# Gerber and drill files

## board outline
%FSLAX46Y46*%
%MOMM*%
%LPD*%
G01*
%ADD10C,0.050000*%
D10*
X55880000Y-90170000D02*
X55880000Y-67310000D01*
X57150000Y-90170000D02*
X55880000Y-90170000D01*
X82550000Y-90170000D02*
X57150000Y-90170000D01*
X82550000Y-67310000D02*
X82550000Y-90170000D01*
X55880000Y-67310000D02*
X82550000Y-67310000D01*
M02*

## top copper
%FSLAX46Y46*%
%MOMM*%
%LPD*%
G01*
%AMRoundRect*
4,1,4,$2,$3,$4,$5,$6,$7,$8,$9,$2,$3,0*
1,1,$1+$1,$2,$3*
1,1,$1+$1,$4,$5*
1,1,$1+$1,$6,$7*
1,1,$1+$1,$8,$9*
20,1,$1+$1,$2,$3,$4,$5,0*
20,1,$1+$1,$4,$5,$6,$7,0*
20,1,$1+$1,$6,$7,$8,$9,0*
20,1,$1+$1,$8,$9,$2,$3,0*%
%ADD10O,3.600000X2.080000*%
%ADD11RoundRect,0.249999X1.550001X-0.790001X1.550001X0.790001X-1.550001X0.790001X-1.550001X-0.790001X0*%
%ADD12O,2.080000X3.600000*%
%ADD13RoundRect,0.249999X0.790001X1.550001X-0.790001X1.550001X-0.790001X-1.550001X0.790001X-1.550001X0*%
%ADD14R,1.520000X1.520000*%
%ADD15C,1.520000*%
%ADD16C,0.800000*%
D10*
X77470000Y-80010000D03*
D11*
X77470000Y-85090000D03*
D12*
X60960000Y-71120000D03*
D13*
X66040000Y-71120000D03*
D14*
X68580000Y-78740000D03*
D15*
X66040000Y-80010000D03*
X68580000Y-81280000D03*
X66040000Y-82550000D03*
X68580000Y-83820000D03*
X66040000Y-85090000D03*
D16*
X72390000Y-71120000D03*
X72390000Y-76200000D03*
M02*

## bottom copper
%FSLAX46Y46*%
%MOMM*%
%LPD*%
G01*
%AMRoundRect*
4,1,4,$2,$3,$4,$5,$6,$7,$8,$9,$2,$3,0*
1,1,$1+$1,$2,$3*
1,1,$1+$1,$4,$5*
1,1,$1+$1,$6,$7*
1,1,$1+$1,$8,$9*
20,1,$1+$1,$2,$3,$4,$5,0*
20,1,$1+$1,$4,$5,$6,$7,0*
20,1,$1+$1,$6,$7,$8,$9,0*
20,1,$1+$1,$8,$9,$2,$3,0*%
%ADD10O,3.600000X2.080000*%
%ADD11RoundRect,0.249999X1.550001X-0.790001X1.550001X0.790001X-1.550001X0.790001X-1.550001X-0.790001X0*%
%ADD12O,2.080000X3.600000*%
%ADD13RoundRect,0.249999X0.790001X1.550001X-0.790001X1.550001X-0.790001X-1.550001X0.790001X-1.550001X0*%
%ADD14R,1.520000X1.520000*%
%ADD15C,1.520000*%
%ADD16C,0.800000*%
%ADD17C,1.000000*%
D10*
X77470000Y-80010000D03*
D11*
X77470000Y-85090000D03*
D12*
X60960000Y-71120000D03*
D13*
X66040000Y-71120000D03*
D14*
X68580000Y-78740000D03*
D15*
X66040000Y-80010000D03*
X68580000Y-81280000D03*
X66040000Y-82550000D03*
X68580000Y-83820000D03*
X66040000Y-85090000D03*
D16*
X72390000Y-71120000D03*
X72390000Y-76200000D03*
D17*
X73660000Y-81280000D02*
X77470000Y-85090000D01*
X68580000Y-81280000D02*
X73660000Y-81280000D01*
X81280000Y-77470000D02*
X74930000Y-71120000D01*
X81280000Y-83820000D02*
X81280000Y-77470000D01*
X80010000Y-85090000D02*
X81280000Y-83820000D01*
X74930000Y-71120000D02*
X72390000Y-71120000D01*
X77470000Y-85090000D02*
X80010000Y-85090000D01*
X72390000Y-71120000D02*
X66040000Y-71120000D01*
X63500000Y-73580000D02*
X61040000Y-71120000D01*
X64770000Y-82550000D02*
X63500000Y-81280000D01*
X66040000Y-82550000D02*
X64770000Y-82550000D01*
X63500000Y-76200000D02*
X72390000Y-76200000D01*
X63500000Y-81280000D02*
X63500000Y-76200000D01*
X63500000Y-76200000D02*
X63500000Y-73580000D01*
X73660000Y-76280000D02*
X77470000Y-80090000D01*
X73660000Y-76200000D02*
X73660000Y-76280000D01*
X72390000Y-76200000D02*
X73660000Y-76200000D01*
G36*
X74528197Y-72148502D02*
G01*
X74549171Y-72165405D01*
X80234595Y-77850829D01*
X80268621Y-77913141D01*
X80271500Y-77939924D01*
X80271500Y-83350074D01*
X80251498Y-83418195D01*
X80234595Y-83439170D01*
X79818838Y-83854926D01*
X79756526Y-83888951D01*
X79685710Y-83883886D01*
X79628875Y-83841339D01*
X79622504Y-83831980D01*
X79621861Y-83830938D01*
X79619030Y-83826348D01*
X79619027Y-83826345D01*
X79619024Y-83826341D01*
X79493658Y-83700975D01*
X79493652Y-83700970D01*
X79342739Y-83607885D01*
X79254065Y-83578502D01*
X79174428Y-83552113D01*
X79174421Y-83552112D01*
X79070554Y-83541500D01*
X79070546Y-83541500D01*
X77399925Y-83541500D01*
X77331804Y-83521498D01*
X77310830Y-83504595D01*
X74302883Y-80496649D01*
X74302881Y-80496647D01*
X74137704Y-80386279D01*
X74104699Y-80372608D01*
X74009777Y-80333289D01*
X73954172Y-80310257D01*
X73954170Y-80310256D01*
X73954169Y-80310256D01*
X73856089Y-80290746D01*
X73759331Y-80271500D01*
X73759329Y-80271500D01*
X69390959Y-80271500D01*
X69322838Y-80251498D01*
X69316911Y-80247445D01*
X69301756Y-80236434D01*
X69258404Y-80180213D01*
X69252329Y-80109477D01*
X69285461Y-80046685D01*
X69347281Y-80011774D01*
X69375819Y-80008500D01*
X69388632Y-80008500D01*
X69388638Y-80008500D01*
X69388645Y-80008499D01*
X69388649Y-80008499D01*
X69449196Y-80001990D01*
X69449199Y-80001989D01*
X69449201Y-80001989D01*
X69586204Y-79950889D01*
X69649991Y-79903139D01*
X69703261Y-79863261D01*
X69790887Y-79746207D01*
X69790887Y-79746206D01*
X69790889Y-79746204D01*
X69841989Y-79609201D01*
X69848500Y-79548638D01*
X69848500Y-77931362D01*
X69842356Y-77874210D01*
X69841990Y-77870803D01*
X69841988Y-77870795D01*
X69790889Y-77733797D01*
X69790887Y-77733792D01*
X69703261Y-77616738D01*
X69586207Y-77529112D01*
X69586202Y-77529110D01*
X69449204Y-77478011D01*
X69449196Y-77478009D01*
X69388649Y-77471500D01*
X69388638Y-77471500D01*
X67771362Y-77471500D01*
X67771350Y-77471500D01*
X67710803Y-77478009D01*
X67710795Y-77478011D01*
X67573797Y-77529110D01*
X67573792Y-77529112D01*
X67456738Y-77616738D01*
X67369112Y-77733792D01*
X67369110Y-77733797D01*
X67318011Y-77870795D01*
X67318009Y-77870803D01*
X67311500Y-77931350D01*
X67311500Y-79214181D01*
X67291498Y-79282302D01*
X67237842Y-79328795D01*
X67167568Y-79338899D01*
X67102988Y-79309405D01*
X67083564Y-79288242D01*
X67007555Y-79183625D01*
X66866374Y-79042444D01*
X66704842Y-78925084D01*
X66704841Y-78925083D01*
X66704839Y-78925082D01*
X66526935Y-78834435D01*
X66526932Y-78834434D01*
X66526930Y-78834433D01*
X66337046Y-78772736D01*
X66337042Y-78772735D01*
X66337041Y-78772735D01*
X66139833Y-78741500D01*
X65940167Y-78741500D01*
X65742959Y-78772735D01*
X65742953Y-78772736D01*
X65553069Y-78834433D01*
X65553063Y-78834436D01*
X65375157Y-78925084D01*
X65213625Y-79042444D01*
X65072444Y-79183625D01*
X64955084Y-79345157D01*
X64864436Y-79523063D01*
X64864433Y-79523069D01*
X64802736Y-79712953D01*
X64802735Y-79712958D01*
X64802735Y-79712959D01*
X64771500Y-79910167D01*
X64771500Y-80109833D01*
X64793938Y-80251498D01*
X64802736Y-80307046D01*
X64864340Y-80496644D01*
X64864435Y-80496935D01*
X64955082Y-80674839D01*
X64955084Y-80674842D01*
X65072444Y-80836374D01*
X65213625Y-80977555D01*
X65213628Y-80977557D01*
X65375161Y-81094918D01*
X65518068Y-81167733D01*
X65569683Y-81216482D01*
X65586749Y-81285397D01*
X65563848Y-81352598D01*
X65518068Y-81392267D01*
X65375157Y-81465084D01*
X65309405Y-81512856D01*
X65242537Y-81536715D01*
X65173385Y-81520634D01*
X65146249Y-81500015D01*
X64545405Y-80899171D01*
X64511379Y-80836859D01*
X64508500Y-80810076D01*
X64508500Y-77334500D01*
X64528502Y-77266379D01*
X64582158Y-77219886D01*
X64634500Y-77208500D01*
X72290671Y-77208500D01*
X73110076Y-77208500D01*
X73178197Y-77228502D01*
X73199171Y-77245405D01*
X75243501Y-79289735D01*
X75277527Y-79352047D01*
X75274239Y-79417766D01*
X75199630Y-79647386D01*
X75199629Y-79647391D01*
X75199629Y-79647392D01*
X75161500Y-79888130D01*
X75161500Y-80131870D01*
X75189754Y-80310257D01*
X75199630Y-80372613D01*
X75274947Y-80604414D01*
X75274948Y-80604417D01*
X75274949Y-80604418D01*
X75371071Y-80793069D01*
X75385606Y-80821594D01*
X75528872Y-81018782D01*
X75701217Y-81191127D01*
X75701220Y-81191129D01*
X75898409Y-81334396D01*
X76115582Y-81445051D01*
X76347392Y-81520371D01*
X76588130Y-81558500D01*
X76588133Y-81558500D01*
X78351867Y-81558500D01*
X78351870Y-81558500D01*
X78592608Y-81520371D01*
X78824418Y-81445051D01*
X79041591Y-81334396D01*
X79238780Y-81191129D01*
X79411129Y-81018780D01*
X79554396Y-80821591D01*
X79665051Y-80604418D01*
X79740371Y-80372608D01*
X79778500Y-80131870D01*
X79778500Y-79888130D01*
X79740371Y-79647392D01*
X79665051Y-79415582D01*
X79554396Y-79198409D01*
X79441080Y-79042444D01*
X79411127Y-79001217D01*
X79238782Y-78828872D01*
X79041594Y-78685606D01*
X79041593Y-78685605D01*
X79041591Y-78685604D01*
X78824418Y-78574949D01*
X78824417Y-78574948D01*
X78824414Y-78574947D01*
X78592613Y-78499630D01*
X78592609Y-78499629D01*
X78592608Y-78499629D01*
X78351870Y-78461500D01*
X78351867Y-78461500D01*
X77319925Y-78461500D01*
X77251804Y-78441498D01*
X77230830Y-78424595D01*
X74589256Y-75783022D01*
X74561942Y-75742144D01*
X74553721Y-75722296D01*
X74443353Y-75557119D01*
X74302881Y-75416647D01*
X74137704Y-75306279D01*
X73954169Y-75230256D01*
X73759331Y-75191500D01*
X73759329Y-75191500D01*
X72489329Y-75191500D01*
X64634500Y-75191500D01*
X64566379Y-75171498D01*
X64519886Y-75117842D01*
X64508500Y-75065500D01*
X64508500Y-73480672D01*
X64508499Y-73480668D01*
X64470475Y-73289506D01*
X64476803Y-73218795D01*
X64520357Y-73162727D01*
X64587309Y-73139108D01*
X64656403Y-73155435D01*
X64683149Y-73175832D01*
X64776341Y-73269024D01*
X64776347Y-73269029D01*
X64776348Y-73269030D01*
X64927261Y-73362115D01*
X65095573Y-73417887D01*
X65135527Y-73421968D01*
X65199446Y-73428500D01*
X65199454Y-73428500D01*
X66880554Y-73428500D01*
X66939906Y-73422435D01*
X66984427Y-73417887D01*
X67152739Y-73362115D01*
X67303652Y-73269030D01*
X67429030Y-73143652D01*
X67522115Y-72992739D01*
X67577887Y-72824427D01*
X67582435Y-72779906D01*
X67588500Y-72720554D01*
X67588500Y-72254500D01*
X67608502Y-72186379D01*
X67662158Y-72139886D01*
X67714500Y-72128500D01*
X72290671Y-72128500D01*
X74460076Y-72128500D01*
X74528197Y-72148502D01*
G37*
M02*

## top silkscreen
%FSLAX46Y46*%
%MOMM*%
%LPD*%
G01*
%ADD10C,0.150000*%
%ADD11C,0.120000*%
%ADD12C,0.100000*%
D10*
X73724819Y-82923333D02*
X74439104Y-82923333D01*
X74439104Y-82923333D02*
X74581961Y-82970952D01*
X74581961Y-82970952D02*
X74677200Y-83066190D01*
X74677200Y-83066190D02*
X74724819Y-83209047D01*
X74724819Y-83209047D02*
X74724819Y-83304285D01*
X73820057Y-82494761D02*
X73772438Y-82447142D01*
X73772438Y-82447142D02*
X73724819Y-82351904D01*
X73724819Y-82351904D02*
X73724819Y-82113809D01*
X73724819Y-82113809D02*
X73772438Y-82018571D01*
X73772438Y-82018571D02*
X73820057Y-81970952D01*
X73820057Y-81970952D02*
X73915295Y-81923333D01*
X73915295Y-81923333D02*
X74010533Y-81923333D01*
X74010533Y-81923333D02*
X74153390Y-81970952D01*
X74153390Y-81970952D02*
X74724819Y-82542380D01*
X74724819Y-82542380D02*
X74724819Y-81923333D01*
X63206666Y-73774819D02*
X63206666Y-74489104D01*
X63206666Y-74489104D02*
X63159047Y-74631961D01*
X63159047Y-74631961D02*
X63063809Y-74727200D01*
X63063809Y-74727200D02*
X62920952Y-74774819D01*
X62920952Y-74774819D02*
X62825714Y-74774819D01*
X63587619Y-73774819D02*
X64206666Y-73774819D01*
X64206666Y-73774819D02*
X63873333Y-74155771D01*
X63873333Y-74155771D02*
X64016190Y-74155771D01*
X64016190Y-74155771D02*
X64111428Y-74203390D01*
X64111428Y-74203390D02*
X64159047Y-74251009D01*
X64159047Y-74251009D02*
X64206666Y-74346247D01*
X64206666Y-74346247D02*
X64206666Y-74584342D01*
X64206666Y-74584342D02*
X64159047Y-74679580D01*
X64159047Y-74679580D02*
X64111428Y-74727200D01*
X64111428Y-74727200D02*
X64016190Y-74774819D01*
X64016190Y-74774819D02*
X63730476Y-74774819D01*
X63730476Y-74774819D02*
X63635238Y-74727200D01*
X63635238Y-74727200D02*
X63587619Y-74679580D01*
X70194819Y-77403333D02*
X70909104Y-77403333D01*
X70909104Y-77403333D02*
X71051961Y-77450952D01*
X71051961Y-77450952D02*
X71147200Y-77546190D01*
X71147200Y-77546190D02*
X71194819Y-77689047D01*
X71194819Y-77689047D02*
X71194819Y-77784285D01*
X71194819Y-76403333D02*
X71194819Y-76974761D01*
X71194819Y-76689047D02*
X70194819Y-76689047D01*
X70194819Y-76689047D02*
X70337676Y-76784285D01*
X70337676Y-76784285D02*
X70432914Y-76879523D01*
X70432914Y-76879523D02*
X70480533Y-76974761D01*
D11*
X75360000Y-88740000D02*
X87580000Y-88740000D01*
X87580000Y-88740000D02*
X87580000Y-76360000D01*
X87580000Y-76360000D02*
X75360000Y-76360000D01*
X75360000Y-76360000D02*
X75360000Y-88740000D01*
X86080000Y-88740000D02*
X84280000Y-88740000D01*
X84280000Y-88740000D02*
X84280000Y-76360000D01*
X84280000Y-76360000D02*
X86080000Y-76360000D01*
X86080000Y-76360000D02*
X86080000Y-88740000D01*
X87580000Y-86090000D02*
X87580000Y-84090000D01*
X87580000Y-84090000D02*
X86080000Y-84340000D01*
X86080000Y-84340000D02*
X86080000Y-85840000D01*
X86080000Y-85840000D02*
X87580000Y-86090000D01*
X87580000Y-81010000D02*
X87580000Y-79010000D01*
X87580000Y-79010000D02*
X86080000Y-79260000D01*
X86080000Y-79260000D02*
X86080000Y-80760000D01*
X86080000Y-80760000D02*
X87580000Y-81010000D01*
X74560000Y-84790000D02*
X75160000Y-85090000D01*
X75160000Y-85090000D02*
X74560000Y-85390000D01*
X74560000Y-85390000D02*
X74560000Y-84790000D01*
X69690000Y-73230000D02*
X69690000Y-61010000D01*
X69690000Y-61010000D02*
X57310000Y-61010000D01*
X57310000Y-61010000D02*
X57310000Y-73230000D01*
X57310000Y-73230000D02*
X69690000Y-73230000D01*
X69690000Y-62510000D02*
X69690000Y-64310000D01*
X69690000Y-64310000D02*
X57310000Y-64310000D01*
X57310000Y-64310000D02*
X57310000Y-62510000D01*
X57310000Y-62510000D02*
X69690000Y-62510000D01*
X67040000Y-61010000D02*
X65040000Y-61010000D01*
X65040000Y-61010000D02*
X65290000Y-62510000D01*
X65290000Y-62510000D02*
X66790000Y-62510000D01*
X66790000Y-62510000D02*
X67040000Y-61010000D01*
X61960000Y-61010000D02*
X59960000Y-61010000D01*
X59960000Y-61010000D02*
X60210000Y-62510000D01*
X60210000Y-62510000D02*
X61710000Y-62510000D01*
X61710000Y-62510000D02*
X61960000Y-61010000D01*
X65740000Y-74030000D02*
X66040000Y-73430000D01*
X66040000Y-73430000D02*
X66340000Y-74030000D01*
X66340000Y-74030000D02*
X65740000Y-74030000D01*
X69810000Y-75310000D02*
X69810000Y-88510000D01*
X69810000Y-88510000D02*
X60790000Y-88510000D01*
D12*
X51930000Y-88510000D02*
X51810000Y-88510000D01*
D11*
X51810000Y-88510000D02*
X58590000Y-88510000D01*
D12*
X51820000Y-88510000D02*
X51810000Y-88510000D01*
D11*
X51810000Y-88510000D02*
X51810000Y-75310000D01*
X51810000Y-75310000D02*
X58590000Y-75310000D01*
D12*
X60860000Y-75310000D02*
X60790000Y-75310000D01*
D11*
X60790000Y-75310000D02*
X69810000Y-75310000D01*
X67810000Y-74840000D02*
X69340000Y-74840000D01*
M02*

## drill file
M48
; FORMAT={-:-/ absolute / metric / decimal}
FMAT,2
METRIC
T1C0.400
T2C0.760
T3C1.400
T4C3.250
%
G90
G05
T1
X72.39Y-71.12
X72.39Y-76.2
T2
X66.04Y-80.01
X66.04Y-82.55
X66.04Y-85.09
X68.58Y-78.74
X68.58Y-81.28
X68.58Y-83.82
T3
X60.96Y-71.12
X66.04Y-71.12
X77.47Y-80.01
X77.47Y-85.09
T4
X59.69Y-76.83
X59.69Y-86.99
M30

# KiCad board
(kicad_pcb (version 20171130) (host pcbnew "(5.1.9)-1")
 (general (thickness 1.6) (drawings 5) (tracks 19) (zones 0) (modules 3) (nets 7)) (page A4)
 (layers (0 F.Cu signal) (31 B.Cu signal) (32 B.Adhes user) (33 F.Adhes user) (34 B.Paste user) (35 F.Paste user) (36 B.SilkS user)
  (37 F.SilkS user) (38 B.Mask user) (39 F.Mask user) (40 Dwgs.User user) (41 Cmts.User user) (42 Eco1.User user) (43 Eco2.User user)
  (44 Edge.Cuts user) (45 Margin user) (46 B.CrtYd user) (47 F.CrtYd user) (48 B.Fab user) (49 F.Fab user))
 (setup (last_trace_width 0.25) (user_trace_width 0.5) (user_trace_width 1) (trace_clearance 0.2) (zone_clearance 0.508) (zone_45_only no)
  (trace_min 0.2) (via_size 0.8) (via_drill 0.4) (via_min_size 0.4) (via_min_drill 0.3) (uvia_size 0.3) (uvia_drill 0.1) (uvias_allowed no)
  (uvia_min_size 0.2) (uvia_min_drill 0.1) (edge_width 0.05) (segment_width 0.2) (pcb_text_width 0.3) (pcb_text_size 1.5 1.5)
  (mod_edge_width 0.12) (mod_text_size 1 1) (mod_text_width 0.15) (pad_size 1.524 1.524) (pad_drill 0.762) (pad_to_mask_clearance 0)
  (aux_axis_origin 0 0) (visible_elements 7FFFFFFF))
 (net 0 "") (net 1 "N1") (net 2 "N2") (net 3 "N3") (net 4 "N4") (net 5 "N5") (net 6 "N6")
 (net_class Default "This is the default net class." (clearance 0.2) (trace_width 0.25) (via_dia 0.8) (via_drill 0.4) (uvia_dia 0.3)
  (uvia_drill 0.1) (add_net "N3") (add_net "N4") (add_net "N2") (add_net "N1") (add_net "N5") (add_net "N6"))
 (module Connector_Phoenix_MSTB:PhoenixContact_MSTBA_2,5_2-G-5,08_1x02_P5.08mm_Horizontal (layer F.Cu) (at 77.47 85.09 90)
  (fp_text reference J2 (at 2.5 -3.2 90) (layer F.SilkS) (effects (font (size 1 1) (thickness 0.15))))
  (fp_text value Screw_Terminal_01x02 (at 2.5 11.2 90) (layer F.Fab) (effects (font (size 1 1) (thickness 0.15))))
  (fp_line (start -3.65 -2.11) (end -3.65 10.11) (layer F.SilkS) (width 0.12))
  (fp_line (start -3.65 10.11) (end 8.73 10.11) (layer F.SilkS) (width 0.12))
  (fp_line (start 8.73 10.11) (end 8.73 -2.11) (layer F.SilkS) (width 0.12))
  (fp_line (start 8.73 -2.11) (end -3.65 -2.11) (layer F.SilkS) (width 0.12))
  (fp_line (start -3.65 8.61) (end -3.65 6.81) (layer F.SilkS) (width 0.12))
  (fp_line (start -3.65 6.81) (end 8.73 6.81) (layer F.SilkS) (width 0.12))
  (fp_line (start 8.73 6.81) (end 8.73 8.61) (layer F.SilkS) (width 0.12))
  (fp_line (start 8.73 8.61) (end -3.65 8.61) (layer F.SilkS) (width 0.12))
  (fp_line (start -1 10.11) (end 1 10.11) (layer F.SilkS) (width 0.12))
  (fp_line (start 1 10.11) (end 0.75 8.61) (layer F.SilkS) (width 0.12))
  (fp_line (start 0.75 8.61) (end -0.75 8.61) (layer F.SilkS) (width 0.12))
  (fp_line (start -0.75 8.61) (end -1 10.11) (layer F.SilkS) (width 0.12))
  (fp_line (start 4.08 10.11) (end 6.08 10.11) (layer F.SilkS) (width 0.12))
  (fp_line (start 6.08 10.11) (end 5.83 8.61) (layer F.SilkS) (width 0.12))
  (fp_line (start 5.83 8.61) (end 4.33 8.61) (layer F.SilkS) (width 0.12))
  (fp_line (start 4.33 8.61) (end 4.08 10.11) (layer F.SilkS) (width 0.12))
  (fp_line (start 0.3 -2.91) (end 0 -2.31) (layer F.SilkS) (width 0.12))
  (fp_line (start 0 -2.31) (end -0.3 -2.91) (layer F.SilkS) (width 0.12))
  (fp_line (start -0.3 -2.91) (end 0.3 -2.91) (layer F.SilkS) (width 0.12))
  (pad 2 thru_hole oval (at 5.08 0 90) (size 2.08 3.6) (drill 1.4) (layers *.Cu *.Mask) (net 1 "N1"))
  (pad 1 thru_hole roundrect (at 0 0 90) (size 2.08 3.6) (drill 1.4) (layers *.Cu *.Mask) (roundrect_rratio 0.120192) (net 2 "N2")))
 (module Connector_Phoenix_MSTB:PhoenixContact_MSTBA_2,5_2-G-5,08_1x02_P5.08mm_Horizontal (layer F.Cu) (at 66.04 71.12 180)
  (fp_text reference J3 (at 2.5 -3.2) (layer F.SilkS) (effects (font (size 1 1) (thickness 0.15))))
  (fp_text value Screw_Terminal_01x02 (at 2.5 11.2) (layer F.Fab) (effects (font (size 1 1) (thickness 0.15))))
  (fp_line (start -3.65 -2.11) (end -3.65 10.11) (layer F.SilkS) (width 0.12))
  (fp_line (start -3.65 10.11) (end 8.73 10.11) (layer F.SilkS) (width 0.12))
  (fp_line (start 8.73 10.11) (end 8.73 -2.11) (layer F.SilkS) (width 0.12))
  (fp_line (start 8.73 -2.11) (end -3.65 -2.11) (layer F.SilkS) (width 0.12))
  (fp_line (start -3.65 8.61) (end -3.65 6.81) (layer F.SilkS) (width 0.12))
  (fp_line (start -3.65 6.81) (end 8.73 6.81) (layer F.SilkS) (width 0.12))
  (fp_line (start 8.73 6.81) (end 8.73 8.61) (layer F.SilkS) (width 0.12))
  (fp_line (start 8.73 8.61) (end -3.65 8.61) (layer F.SilkS) (width 0.12))
  (fp_line (start -1 10.11) (end 1 10.11) (layer F.SilkS) (width 0.12))
  (fp_line (start 1 10.11) (end 0.75 8.61) (layer F.SilkS) (width 0.12))
  (fp_line (start 0.75 8.61) (end -0.75 8.61) (layer F.SilkS) (width 0.12))
  (fp_line (start -0.75 8.61) (end -1 10.11) (layer F.SilkS) (width 0.12))
  (fp_line (start 4.08 10.11) (end 6.08 10.11) (layer F.SilkS) (width 0.12))
  (fp_line (start 6.08 10.11) (end 5.83 8.61) (layer F.SilkS) (width 0.12))
  (fp_line (start 5.83 8.61) (end 4.33 8.61) (layer F.SilkS) (width 0.12))
  (fp_line (start 4.33 8.61) (end 4.08 10.11) (layer F.SilkS) (width 0.12))
  (fp_line (start 0.3 -2.91) (end 0 -2.31) (layer F.SilkS) (width 0.12))
  (fp_line (start 0 -2.31) (end -0.3 -2.91) (layer F.SilkS) (width 0.12))
  (fp_line (start -0.3 -2.91) (end 0.3 -2.91) (layer F.SilkS) (width 0.12))
  (pad 2 thru_hole oval (at 5.08 0 180) (size 2.08 3.6) (drill 1.4) (layers *.Cu *.Mask) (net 1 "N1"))
  (pad 1 thru_hole roundrect (at 0 0 180) (size 2.08 3.6) (drill 1.4) (layers *.Cu *.Mask) (roundrect_rratio 0.120192) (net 2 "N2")))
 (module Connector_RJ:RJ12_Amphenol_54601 (layer F.Cu) (at 68.58 78.74 270)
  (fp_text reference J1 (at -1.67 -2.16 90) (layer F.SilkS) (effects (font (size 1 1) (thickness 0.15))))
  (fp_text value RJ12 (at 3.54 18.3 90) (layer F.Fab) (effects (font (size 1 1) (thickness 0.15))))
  (fp_line (start -3.43 -1.23) (end 9.77 -1.23) (layer F.SilkS) (width 0.12))
  (fp_line (start 9.77 -1.23) (end 9.77 7.79) (layer F.SilkS) (width 0.12))
  (fp_line (start 9.77 16.65) (end 9.77 16.77) (layer F.SilkS) (width 0.1))
  (fp_line (start 9.77 16.77) (end 9.77 9.99) (layer F.SilkS) (width 0.12))
  (fp_line (start 9.77 16.76) (end 9.77 16.77) (layer F.SilkS) (width 0.1))
  (fp_line (start 9.77 16.77) (end -3.43 16.77) (layer F.SilkS) (width 0.12))
  (fp_line (start -3.43 16.77) (end -3.43 9.99) (layer F.SilkS) (width 0.12))
  (fp_line (start -3.43 7.72) (end -3.43 7.79) (layer F.SilkS) (width 0.1))
  (fp_line (start -3.43 7.79) (end -3.43 -1.23) (layer F.SilkS) (width 0.12))
  (fp_line (start -3.9 0.77) (end -3.9 -0.76) (layer F.SilkS) (width 0.12))
  (pad 1 thru_hole rect (at 0 0 270) (size 1.52 1.52) (drill 0.76) (layers *.Cu *.Mask) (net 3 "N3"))
  (pad "" np_thru_hole circle (at -1.91 8.89 270) (size 3.25 3.25) (drill 3.25) (layers *.Cu *.Mask))
  (pad 2 thru_hole circle (at 1.27 2.54 270) (size 1.52 1.52) (drill 0.76) (layers *.Cu *.Mask) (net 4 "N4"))
  (pad 3 thru_hole circle (at 2.54 0 270) (size 1.52 1.52) (drill 0.76) (layers *.Cu *.Mask) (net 2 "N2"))
  (pad 4 thru_hole circle (at 3.81 2.54 270) (size 1.52 1.52) (drill 0.76) (layers *.Cu *.Mask) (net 1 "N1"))
  (pad 5 thru_hole circle (at 5.08 0 270) (size 1.52 1.52) (drill 0.76) (layers *.Cu *.Mask) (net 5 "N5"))
  (pad 6 thru_hole circle (at 6.35 2.54 270) (size 1.52 1.52) (drill 0.76) (layers *.Cu *.Mask) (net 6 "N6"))
  (pad "" np_thru_hole circle (at 8.25 8.89 270) (size 3.25 3.25) (drill 3.25) (layers *.Cu *.Mask)))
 (gr_line (start 55.88 90.17) (end 55.88 67.31) (layer Edge.Cuts) (width 0.05))
 (gr_line (start 57.15 90.17) (end 55.88 90.17) (layer Edge.Cuts) (width 0.05))
 (gr_line (start 82.55 90.17) (end 57.15 90.17) (layer Edge.Cuts) (width 0.05))
 (gr_line (start 82.55 67.31) (end 82.55 90.17) (layer Edge.Cuts) (width 0.05))
 (gr_line (start 55.88 67.31) (end 82.55 67.31) (layer Edge.Cuts) (width 0.05))
 (segment (start 73.66 81.28) (end 77.47 85.09) (width 1) (layer B.Cu) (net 2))
 (segment (start 68.58 81.28) (end 73.66 81.28) (width 1) (layer B.Cu) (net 2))
 (segment (start 81.28 77.47) (end 74.93 71.12) (width 1) (layer B.Cu) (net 2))
 (segment (start 81.28 83.82) (end 81.28 77.47) (width 1) (layer B.Cu) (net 2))
 (segment (start 80.01 85.09) (end 81.28 83.82) (width 1) (layer B.Cu) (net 2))
 (segment (start 74.93 71.12) (end 72.39 71.12) (width 1) (layer B.Cu) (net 2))
 (segment (start 77.47 85.09) (end 80.01 85.09) (width 1) (layer B.Cu) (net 2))
 (segment (start 72.39 71.12) (end 66.04 71.12) (width 1) (layer B.Cu) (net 2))
 (via (at 72.39 71.12) (size 0.8) (drill 0.4) (layers F.Cu B.Cu) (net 2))
 (segment (start 63.5 73.58) (end 61.04 71.12) (width 1) (layer B.Cu) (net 1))
 (segment (start 64.77 82.55) (end 63.5 81.28) (width 1) (layer B.Cu) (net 1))
 (segment (start 66.04 82.55) (end 64.77 82.55) (width 1) (layer B.Cu) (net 1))
 (segment (start 63.5 76.2) (end 72.39 76.2) (width 1) (layer B.Cu) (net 1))
 (segment (start 63.5 81.28) (end 63.5 76.2) (width 1) (layer B.Cu) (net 1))
 (segment (start 63.5 76.2) (end 63.5 73.58) (width 1) (layer B.Cu) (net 1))
 (segment (start 73.66 76.28) (end 77.47 80.09) (width 1) (layer B.Cu) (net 1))
 (segment (start 73.66 76.2) (end 73.66 76.28) (width 1) (layer B.Cu) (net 1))
 (segment (start 72.39 76.2) (end 73.66 76.2) (width 1) (layer B.Cu) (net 1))
 (via (at 72.39 76.2) (size 0.8) (drill 0.4) (layers F.Cu B.Cu) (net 1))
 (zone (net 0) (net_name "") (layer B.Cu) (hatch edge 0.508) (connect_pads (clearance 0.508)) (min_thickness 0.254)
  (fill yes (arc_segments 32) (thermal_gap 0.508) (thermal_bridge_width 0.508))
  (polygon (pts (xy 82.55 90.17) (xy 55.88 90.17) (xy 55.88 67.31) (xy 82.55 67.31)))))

